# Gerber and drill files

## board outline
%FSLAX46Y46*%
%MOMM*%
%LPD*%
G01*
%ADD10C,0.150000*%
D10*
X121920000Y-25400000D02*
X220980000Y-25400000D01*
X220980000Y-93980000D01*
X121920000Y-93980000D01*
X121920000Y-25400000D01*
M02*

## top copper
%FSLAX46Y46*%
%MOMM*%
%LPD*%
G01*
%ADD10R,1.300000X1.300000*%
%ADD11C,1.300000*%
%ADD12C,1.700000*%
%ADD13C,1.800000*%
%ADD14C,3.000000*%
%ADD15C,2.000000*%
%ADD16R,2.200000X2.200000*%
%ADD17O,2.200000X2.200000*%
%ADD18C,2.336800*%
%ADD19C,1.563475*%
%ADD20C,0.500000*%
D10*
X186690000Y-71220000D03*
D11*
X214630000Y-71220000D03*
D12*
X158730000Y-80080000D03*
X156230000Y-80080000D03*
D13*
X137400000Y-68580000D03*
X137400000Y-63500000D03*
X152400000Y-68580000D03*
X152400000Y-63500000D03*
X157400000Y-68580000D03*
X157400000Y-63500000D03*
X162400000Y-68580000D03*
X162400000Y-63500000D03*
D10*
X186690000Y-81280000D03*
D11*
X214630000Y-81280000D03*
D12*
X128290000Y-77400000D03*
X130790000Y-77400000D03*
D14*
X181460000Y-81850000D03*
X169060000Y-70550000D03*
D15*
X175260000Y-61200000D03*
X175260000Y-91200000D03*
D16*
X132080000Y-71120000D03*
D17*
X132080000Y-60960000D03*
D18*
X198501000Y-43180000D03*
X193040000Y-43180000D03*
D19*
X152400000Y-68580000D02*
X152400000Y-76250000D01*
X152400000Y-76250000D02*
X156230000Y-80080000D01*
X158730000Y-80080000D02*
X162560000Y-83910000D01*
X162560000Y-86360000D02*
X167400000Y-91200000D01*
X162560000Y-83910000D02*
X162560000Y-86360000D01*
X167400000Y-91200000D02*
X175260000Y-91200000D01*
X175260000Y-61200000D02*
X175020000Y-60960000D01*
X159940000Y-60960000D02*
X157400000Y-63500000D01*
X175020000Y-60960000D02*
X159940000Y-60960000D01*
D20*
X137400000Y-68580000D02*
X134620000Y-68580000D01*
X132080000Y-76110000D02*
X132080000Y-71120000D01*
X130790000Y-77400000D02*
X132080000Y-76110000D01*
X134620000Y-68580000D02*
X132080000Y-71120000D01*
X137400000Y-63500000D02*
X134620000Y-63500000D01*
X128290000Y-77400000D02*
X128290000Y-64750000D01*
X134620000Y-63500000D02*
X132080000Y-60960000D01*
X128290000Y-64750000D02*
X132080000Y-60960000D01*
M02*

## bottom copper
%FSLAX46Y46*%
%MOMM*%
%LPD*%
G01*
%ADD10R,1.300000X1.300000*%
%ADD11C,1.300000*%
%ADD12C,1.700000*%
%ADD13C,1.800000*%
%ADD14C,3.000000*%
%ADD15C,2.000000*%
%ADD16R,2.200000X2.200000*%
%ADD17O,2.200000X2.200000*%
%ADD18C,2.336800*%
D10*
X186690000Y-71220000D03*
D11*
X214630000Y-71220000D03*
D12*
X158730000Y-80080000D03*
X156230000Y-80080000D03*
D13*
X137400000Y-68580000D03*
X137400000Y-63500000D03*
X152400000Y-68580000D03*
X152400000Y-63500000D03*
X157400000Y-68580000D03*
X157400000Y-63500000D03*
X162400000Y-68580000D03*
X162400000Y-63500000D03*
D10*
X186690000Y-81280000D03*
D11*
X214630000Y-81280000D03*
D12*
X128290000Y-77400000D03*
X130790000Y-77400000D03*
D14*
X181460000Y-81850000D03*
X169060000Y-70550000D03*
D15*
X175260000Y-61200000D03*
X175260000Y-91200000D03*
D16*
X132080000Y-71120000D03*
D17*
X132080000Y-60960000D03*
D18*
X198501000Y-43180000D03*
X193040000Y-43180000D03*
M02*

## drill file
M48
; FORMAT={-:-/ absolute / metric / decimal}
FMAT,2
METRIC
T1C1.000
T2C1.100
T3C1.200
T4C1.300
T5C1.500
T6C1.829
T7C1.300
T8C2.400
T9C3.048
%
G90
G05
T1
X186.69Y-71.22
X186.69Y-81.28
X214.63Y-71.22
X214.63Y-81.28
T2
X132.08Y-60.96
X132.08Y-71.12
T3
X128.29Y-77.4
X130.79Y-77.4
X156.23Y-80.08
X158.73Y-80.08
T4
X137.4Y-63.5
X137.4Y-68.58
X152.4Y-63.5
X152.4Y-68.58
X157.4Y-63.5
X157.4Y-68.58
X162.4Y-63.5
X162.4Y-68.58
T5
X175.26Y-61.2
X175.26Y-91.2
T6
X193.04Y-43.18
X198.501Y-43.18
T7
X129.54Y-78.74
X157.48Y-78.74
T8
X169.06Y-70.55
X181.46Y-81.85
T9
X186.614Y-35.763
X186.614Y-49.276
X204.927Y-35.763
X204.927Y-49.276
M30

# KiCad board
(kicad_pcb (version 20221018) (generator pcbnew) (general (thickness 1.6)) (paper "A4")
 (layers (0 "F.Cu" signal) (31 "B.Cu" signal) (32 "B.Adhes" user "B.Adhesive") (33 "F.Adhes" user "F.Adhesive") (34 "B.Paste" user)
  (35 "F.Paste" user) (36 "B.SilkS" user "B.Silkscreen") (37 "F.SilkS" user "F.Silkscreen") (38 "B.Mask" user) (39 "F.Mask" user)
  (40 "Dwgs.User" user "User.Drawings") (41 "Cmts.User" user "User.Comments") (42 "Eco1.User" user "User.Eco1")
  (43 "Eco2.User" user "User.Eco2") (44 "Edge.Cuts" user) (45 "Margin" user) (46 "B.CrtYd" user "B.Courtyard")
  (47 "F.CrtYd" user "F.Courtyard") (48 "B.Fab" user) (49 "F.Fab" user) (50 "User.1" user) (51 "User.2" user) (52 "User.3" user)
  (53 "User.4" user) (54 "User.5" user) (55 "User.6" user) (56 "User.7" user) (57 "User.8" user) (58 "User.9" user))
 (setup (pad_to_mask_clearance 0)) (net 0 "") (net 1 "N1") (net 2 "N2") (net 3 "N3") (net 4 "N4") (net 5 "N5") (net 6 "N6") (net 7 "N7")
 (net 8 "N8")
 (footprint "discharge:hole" (layer "F.Cu") (at 0.25 0.25)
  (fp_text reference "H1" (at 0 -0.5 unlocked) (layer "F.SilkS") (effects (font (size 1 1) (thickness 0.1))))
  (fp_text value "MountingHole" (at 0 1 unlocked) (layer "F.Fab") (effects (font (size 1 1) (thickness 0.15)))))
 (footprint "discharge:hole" (layer "F.Cu") (at 0.25 3.25)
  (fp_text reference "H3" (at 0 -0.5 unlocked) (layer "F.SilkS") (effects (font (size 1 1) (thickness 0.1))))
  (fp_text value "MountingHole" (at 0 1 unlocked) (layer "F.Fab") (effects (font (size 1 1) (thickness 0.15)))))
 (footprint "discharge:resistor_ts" (layer "F.Cu") (at 190.627 67.4735)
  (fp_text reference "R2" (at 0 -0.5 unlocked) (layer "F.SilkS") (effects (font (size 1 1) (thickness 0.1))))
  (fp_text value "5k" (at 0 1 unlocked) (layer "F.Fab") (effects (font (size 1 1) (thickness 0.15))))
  (pad "1" thru_hole rect (at -3.937 3.7465) (size 1.3 1.3) (drill 1) (layers "*.Cu" "*.Mask") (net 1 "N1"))
  (pad "2" thru_hole circle (at 24.003 3.7465) (size 1.3 1.3) (drill 1) (layers "*.Cu" "*.Mask") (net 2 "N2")))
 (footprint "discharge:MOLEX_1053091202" (layer "F.Cu") (at 158.73 80.08 180)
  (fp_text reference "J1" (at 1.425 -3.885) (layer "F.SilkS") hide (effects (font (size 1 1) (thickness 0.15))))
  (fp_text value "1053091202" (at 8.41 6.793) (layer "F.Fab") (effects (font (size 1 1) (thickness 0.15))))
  (pad "" np_thru_hole circle (at 1.25 1.34 180) (size 1.3 1.3) (drill 1.3) (layers "*.Cu" "*.Mask"))
  (pad "1" thru_hole circle (at 0 0 180) (size 1.7 1.7) (drill 1.2) (layers "*.Cu") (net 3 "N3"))
  (pad "2" thru_hole circle (at 2.5 0 180) (size 1.7 1.7) (drill 1.2) (layers "*.Cu") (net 2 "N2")))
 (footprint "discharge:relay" (layer "F.Cu") (at 134.68 72.39 90)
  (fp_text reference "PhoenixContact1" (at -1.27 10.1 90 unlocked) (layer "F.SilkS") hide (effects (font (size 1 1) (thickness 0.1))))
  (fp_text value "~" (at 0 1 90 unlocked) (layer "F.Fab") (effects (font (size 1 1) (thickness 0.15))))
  (pad "1" thru_hole circle (at 3.81 2.72 90) (size 1.8 1.8) (drill 1.3) (layers "*.Cu" "*.Mask") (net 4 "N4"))
  (pad "2" thru_hole circle (at 8.89 2.72 90) (size 1.8 1.8) (drill 1.3) (layers "*.Cu" "*.Mask") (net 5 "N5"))
  (pad "3" thru_hole circle (at 3.81 17.72 90) (size 1.8 1.8) (drill 1.3) (layers "*.Cu" "*.Mask") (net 2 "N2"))
  (pad "3" thru_hole circle (at 8.89 17.72 90) (size 1.8 1.8) (drill 1.3) (layers "*.Cu" "*.Mask") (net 2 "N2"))
  (pad "4" thru_hole circle (at 3.81 22.72 90) (size 1.8 1.8) (drill 1.3) (layers "*.Cu" "*.Mask") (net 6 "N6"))
  (pad "4" thru_hole circle (at 8.89 22.72 90) (size 1.8 1.8) (drill 1.3) (layers "*.Cu" "*.Mask") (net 6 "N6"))
  (pad "5" thru_hole circle (at 3.81 27.72 90) (size 1.8 1.8) (drill 1.3) (layers "*.Cu" "*.Mask") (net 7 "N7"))
  (pad "5" thru_hole circle (at 8.89 27.72 90) (size 1.8 1.8) (drill 1.3) (layers "*.Cu" "*.Mask") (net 7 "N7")))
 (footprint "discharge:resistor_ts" (layer "F.Cu") (at 190.627 77.5335)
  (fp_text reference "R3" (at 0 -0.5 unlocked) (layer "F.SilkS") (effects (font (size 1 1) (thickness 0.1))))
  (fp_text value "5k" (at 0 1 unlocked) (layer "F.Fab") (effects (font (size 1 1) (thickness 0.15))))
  (pad "1" thru_hole rect (at -3.937 3.7465) (size 1.3 1.3) (drill 1) (layers "*.Cu" "*.Mask") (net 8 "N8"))
  (pad "2" thru_hole circle (at 24.003 3.7465) (size 1.3 1.3) (drill 1) (layers "*.Cu" "*.Mask") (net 3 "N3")))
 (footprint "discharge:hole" (layer "F.Cu") (at 0.25 1.75)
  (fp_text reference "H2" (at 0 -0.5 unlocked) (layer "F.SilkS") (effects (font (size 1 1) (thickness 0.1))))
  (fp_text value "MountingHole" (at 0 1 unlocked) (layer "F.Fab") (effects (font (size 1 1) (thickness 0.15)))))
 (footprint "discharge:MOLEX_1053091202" (layer "F.Cu") (at 128.29 77.4)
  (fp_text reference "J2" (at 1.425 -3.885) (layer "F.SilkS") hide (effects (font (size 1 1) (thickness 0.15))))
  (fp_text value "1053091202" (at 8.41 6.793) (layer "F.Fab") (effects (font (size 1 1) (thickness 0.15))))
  (pad "" np_thru_hole circle (at 1.25 1.34) (size 1.3 1.3) (drill 1.3) (layers "*.Cu" "*.Mask"))
  (pad "1" thru_hole circle (at 0 0) (size 1.7 1.7) (drill 1.2) (layers "*.Cu") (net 5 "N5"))
  (pad "2" thru_hole circle (at 2.5 0) (size 1.7 1.7) (drill 1.2) (layers "*.Cu") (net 4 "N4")))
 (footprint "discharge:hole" (layer "F.Cu") (at 0.25 4.75)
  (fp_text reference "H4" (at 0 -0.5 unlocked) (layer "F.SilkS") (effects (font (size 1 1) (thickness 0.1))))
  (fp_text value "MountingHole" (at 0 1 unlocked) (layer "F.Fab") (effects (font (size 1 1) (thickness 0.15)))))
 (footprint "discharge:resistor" (layer "F.Cu") (at 166.76 84.7 90)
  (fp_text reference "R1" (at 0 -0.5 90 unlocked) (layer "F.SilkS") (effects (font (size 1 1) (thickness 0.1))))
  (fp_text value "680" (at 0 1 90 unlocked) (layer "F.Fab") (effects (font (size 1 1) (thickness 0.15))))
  (pad "" np_thru_hole circle (at 2.85 14.7 90) (size 3 3) (drill 2.4) (layers "F&B.Cu" "*.Mask"))
  (pad "" np_thru_hole circle (at 14.15 2.3 90) (size 3 3) (drill 2.4) (layers "F&B.Cu" "*.Mask"))
  (pad "1" thru_hole circle (at 23.5 8.5 90) (size 2 2) (drill 1.5) (layers "*.Cu" "*.Mask") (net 6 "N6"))
  (pad "2" thru_hole circle (at -6.5 8.5 90) (size 2 2) (drill 1.5) (layers "*.Cu" "*.Mask") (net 3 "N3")))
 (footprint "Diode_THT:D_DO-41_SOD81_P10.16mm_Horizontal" (layer "F.Cu") (at 132.08 71.12 90)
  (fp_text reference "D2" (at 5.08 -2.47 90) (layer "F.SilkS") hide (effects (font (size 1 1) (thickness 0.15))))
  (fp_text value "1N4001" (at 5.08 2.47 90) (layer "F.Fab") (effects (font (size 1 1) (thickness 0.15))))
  (pad "1" thru_hole rect (at 0 0 90) (size 2.2 2.2) (drill 1.1) (layers "*.Cu" "*.Mask") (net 4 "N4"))
  (pad "2" thru_hole oval (at 10.16 0 90) (size 2.2 2.2) (drill 1.1) (layers "*.Cu" "*.Mask") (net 5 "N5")))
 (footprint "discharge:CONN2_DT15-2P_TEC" (layer "F.Cu") (at 193.04 43.18)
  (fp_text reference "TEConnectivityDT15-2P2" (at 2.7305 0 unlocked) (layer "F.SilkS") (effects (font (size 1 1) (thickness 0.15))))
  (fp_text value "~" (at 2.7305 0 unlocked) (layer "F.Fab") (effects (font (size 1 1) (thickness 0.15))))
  (pad "" np_thru_hole circle (at -6.4262 -7.4168) (size 3.048 3.048) (drill 3.048) (layers))
  (pad "" np_thru_hole circle (at -6.4262 6.096) (size 3.048 3.048) (drill 3.048) (layers))
  (pad "" np_thru_hole circle (at 11.8872 -7.4168) (size 3.048 3.048) (drill 3.048) (layers))
  (pad "" np_thru_hole circle (at 11.8872 6.096) (size 3.048 3.048) (drill 3.048) (layers))
  (pad "1" thru_hole circle (at 5.461 0) (size 2.3368 2.3368) (drill 1.8288) (layers "*.Cu" "*.Mask") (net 8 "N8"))
  (pad "2" thru_hole circle (at 0 0) (size 2.3368 2.3368) (drill 1.8288) (layers "*.Cu" "*.Mask") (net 1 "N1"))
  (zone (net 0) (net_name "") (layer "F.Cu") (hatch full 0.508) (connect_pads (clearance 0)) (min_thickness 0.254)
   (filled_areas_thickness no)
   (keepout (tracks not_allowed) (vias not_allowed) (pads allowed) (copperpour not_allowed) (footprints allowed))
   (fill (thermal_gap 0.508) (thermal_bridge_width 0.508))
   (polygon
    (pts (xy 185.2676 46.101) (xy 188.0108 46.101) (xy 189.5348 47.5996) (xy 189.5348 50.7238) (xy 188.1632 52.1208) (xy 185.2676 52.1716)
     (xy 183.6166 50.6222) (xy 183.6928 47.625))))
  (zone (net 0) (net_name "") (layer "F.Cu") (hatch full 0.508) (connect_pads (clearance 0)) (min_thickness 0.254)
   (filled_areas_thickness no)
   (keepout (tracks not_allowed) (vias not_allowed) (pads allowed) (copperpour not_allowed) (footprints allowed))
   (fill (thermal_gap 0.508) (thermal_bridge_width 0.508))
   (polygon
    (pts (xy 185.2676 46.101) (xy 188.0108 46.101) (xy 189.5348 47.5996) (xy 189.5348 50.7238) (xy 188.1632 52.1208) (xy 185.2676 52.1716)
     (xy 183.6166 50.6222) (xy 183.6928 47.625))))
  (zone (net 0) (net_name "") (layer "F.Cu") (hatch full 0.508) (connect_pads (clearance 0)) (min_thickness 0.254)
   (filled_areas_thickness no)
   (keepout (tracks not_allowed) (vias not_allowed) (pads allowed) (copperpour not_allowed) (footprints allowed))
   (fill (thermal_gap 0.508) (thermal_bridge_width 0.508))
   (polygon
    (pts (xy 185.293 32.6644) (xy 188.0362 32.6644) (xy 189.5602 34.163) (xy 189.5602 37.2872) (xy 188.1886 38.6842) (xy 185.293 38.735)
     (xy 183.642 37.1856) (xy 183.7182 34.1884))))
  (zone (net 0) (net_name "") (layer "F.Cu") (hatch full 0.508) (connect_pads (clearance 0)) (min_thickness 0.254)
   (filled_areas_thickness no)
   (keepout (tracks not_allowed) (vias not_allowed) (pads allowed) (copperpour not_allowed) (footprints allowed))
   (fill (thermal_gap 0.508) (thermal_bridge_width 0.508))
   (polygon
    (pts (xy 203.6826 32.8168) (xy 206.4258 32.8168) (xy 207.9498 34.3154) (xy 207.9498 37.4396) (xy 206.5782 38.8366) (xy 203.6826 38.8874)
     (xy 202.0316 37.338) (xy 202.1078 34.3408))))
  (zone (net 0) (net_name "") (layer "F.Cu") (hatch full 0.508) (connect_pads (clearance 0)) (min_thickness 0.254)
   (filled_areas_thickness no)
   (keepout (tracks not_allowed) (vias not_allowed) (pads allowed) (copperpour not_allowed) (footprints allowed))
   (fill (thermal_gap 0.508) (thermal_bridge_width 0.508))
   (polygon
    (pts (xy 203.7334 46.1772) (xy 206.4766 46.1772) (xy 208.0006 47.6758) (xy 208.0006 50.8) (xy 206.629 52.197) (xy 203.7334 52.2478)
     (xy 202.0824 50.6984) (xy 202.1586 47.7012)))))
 (gr_rect (start 121.92 25.4) (end 220.98 93.98) (stroke (width 0.15) (type default)) (fill none) (layer "Edge.Cuts"))
 (segment (start 152.4 68.58) (end 152.4 76.25) (width 1.563475) (layer "F.Cu") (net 2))
 (segment (start 152.4 76.25) (end 156.23 80.08) (width 1.563475) (layer "F.Cu") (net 2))
 (segment (start 158.73 80.08) (end 162.56 83.91) (width 1.563475) (layer "F.Cu") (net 3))
 (segment (start 162.56 86.36) (end 167.4 91.2) (width 1.563475) (layer "F.Cu") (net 3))
 (segment (start 162.56 83.91) (end 162.56 86.36) (width 1.563475) (layer "F.Cu") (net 3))
 (segment (start 167.4 91.2) (end 175.26 91.2) (width 1.563475) (layer "F.Cu") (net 3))
 (segment (start 175.26 61.2) (end 175.02 60.96) (width 1.563475) (layer "F.Cu") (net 6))
 (segment (start 159.94 60.96) (end 157.4 63.5) (width 1.563475) (layer "F.Cu") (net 6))
 (segment (start 175.02 60.96) (end 159.94 60.96) (width 1.563475) (layer "F.Cu") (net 6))
 (segment (start 137.4 68.58) (end 134.62 68.58) (width 0.5) (layer "F.Cu") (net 4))
 (segment (start 132.08 76.11) (end 132.08 71.12) (width 0.5) (layer "F.Cu") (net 4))
 (segment (start 130.79 77.4) (end 132.08 76.11) (width 0.5) (layer "F.Cu") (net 4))
 (segment (start 134.62 68.58) (end 132.08 71.12) (width 0.5) (layer "F.Cu") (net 4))
 (segment (start 137.4 63.5) (end 134.62 63.5) (width 0.5) (layer "F.Cu") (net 5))
 (segment (start 128.29 77.4) (end 128.29 64.75) (width 0.5) (layer "F.Cu") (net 5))
 (segment (start 134.62 63.5) (end 132.08 60.96) (width 0.5) (layer "F.Cu") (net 5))
 (segment (start 128.29 64.75) (end 132.08 60.96) (width 0.5) (layer "F.Cu") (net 5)))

